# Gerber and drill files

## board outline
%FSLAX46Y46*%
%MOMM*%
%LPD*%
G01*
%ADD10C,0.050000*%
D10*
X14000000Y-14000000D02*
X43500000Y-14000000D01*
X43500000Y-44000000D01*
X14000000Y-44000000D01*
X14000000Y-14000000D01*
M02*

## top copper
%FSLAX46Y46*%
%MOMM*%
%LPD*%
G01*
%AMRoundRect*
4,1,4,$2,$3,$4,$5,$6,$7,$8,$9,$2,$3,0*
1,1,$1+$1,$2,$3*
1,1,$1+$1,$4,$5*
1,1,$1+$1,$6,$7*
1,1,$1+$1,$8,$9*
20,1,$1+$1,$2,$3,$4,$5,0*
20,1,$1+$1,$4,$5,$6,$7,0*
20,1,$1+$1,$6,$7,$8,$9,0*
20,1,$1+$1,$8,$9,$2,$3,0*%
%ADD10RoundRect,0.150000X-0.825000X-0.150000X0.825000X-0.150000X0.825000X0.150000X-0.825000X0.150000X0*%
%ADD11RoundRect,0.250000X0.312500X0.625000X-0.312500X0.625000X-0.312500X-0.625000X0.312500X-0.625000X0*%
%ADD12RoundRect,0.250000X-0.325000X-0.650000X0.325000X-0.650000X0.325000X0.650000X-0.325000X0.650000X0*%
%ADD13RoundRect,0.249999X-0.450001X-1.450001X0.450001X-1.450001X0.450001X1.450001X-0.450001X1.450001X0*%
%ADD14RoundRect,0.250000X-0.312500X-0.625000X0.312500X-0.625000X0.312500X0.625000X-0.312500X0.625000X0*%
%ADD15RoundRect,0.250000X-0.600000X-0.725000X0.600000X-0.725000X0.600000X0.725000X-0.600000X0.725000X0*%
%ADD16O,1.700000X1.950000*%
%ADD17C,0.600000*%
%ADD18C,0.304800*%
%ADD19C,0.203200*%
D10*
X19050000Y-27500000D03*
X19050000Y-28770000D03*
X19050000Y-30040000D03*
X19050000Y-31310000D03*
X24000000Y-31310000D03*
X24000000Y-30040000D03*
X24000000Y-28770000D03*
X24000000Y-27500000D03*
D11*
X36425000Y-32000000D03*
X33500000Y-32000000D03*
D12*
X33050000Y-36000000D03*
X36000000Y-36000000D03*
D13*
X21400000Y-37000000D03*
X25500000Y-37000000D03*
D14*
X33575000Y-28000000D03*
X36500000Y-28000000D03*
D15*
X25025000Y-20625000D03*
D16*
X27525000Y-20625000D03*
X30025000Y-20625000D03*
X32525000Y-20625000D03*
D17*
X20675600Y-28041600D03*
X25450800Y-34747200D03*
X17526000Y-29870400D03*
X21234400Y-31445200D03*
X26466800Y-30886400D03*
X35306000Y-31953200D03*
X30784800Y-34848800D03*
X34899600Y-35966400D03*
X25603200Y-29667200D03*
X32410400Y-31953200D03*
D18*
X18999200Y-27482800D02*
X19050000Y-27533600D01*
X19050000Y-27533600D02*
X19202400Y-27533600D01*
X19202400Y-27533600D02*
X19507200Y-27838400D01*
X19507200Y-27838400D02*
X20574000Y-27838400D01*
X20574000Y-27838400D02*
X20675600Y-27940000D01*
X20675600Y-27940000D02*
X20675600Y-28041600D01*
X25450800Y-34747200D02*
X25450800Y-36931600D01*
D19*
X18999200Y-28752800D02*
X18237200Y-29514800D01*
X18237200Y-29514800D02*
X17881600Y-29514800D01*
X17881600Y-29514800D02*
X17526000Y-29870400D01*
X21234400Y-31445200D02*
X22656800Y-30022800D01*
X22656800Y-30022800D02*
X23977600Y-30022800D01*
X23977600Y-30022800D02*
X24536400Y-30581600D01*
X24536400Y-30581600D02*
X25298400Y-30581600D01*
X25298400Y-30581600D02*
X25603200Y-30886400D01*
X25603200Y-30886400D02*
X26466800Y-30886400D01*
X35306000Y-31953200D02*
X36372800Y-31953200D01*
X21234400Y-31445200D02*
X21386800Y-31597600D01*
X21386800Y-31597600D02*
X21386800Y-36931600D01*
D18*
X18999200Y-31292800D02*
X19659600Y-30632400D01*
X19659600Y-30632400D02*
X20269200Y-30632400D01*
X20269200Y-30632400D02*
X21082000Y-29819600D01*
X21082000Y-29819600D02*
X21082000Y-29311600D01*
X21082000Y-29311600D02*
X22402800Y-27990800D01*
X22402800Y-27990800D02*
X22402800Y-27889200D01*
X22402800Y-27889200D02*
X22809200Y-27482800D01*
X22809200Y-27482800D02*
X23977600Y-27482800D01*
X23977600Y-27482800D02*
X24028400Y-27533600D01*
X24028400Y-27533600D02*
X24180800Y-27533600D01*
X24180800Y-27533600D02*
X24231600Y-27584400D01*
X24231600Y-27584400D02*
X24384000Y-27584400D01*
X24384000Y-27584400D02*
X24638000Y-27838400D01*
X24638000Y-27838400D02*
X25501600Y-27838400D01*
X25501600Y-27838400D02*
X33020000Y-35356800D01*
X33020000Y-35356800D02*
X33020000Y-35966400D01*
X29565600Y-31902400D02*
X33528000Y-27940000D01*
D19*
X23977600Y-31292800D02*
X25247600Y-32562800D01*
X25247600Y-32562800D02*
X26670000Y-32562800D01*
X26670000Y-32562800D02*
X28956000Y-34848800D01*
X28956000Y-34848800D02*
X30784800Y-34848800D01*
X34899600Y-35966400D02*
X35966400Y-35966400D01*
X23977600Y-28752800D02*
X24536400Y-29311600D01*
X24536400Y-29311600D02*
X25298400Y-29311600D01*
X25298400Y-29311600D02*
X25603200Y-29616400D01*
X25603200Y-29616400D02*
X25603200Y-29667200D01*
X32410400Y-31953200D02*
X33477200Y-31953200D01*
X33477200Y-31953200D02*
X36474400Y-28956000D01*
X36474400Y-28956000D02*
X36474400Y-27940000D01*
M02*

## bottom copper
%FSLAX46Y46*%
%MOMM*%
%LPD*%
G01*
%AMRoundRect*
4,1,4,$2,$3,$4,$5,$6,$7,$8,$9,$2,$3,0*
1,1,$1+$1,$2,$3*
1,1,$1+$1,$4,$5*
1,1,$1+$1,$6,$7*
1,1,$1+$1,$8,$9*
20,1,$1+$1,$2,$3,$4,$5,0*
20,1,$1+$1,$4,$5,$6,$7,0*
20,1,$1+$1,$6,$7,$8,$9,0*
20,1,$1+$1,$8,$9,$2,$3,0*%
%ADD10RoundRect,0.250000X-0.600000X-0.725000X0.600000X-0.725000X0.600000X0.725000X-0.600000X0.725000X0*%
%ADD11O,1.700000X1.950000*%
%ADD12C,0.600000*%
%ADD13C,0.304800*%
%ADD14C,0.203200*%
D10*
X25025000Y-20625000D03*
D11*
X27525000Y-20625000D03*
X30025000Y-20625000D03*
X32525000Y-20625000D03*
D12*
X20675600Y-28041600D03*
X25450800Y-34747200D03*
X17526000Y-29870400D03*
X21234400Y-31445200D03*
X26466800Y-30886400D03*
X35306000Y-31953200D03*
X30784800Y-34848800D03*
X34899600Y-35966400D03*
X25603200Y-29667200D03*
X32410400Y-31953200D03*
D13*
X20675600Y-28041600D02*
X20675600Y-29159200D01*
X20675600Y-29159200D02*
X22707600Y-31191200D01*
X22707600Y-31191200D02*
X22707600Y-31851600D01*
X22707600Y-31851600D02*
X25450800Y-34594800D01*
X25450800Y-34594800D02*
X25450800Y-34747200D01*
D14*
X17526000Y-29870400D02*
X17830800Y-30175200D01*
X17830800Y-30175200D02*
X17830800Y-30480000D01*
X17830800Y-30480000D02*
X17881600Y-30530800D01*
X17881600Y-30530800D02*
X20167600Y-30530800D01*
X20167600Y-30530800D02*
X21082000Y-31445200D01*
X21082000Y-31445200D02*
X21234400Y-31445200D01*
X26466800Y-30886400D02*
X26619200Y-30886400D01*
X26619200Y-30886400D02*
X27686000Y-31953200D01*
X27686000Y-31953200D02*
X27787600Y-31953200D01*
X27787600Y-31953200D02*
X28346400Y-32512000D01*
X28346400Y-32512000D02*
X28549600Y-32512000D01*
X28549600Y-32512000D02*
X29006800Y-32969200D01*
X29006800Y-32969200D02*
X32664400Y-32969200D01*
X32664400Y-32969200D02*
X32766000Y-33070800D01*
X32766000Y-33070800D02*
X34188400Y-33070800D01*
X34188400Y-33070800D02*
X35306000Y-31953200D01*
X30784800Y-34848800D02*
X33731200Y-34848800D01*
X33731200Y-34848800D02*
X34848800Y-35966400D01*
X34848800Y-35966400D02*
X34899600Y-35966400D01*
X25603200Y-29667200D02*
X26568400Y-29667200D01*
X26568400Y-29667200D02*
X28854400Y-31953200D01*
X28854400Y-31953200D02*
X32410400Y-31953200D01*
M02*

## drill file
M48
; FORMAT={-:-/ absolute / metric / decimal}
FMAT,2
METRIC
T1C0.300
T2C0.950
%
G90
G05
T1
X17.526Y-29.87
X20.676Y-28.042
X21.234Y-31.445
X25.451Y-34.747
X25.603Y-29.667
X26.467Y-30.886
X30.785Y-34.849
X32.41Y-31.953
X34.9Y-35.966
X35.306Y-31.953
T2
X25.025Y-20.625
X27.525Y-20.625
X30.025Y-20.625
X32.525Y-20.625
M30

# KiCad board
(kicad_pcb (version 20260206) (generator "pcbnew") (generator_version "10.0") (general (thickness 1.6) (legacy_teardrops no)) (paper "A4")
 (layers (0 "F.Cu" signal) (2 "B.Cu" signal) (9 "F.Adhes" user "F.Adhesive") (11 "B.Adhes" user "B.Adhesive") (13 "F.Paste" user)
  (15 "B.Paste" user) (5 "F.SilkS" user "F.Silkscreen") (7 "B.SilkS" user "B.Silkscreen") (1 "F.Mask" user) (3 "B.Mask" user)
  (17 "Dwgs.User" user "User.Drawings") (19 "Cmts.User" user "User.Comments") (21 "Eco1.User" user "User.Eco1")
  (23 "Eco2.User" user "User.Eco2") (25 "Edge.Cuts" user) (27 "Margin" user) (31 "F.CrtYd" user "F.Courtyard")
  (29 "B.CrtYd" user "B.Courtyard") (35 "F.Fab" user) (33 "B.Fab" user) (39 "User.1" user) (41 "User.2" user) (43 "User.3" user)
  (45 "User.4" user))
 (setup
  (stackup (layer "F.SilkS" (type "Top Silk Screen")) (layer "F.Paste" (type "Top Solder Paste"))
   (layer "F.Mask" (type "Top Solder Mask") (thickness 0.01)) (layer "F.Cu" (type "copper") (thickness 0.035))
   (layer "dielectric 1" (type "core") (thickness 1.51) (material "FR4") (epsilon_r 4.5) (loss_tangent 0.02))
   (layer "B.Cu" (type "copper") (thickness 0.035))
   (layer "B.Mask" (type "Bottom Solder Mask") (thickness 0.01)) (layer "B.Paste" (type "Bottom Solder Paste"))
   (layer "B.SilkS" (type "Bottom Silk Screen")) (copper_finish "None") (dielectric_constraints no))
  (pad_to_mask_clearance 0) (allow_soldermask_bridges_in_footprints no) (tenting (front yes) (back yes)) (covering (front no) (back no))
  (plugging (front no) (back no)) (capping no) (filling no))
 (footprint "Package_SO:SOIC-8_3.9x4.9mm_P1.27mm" (layer "F.Cu") (at 21.525 29.405)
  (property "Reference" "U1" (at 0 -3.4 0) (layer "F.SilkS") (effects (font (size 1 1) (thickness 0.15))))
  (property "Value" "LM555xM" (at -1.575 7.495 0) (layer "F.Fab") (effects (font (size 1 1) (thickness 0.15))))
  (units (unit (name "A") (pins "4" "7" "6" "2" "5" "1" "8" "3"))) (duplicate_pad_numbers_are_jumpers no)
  (pad "1" smd roundrect (at -2.475 -1.905) (size 1.95 0.6) (layers "F.Cu" "F.Mask" "F.Paste") (roundrect_rratio 0.25) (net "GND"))
  (pad "2" smd roundrect (at -2.475 -0.635) (size 1.95 0.6) (layers "F.Cu" "F.Mask" "F.Paste") (roundrect_rratio 0.25)
   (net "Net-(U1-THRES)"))
  (pad "3" smd roundrect (at -2.475 0.635) (size 1.95 0.6) (layers "F.Cu" "F.Mask" "F.Paste") (roundrect_rratio 0.25) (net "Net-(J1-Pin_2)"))
  (pad "4" smd roundrect (at -2.475 1.905) (size 1.95 0.6) (layers "F.Cu" "F.Mask" "F.Paste") (roundrect_rratio 0.25) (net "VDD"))
  (pad "5" smd roundrect (at 2.475 1.905) (size 1.95 0.6) (layers "F.Cu" "F.Mask" "F.Paste") (roundrect_rratio 0.25) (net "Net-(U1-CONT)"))
  (pad "6" smd roundrect (at 2.475 0.635) (size 1.95 0.6) (layers "F.Cu" "F.Mask" "F.Paste") (roundrect_rratio 0.25) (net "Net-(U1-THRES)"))
  (pad "7" smd roundrect (at 2.475 -0.635) (size 1.95 0.6) (layers "F.Cu" "F.Mask" "F.Paste") (roundrect_rratio 0.25) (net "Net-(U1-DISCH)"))
  (pad "8" smd roundrect (at 2.475 -1.905) (size 1.95 0.6) (layers "F.Cu" "F.Mask" "F.Paste") (roundrect_rratio 0.25) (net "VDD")))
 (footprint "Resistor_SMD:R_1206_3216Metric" (layer "F.Cu") (at 34.9625 32 180)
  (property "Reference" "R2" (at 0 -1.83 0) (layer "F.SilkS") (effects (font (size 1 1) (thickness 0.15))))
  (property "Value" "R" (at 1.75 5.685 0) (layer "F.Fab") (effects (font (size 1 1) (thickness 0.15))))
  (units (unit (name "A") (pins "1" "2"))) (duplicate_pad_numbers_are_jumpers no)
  (pad "1" smd roundrect (at -1.4625 0 180) (size 1.125 1.75) (layers "F.Cu" "F.Mask" "F.Paste") (roundrect_rratio 0.222222)
   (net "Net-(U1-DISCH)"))
  (pad "2" smd roundrect (at 1.4625 0 180) (size 1.125 1.75) (layers "F.Cu" "F.Mask" "F.Paste") (roundrect_rratio 0.222222)
   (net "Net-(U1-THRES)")))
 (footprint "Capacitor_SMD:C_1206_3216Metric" (layer "F.Cu") (at 34.525 36)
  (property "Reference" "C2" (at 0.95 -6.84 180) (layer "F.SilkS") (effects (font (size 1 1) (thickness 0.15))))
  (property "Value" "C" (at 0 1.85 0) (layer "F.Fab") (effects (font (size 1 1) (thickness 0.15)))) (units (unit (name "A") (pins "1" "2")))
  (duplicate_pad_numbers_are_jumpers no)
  (pad "1" smd roundrect (at -1.475 0) (size 1.15 1.8) (layers "F.Cu" "F.Mask" "F.Paste") (roundrect_rratio 0.217391) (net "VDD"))
  (pad "2" smd roundrect (at 1.475 0) (size 1.15 1.8) (layers "F.Cu" "F.Mask" "F.Paste") (roundrect_rratio 0.217391) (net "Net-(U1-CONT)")))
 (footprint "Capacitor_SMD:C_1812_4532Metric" (layer "F.Cu") (at 23.45 37)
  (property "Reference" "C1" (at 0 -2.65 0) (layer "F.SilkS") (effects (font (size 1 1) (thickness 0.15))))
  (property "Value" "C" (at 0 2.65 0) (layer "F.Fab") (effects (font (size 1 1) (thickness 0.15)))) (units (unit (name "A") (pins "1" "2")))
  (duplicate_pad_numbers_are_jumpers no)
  (pad "1" smd roundrect (at -2.05 0) (size 1.4 3.4) (layers "F.Cu" "F.Mask" "F.Paste") (roundrect_rratio 0.178571) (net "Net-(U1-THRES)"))
  (pad "2" smd roundrect (at 2.05 0) (size 1.4 3.4) (layers "F.Cu" "F.Mask" "F.Paste") (roundrect_rratio 0.178571) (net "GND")))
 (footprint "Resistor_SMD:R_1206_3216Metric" (layer "F.Cu") (at 35.0375 28)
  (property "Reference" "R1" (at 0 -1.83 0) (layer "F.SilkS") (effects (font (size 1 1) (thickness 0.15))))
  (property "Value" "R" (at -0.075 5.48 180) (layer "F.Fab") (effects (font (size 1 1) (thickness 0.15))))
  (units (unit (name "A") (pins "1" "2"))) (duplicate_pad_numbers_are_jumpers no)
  (pad "1" smd roundrect (at -1.4625 0) (size 1.125 1.75) (layers "F.Cu" "F.Mask" "F.Paste") (roundrect_rratio 0.222222) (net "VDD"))
  (pad "2" smd roundrect (at 1.4625 0) (size 1.125 1.75) (layers "F.Cu" "F.Mask" "F.Paste") (roundrect_rratio 0.222222)
   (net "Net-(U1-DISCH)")))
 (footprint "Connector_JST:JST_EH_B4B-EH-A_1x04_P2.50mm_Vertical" (layer "F.Cu") (at 25.025 20.625)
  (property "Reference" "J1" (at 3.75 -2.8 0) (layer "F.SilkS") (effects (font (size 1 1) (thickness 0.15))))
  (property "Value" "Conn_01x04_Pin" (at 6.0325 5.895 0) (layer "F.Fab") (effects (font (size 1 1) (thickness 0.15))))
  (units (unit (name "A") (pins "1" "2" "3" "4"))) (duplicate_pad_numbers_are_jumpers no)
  (pad "1" thru_hole roundrect (at 0 0) (size 1.7 1.95) (drill 0.95) (layers "*.Cu" "*.Mask") (remove_unused_layers no)
   (roundrect_rratio 0.147059) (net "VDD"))
  (pad "2" thru_hole oval (at 2.5 0) (size 1.7 1.95) (drill 0.95) (layers "*.Cu" "*.Mask") (remove_unused_layers no) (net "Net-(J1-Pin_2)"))
  (pad "3" thru_hole oval (at 5 0) (size 1.7 1.95) (drill 0.95) (layers "*.Cu" "*.Mask") (remove_unused_layers no)
   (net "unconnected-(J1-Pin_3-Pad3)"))
  (pad "4" thru_hole oval (at 7.5 0) (size 1.7 1.95) (drill 0.95) (layers "*.Cu" "*.Mask") (remove_unused_layers no) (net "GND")))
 (gr_rect (start 14 14) (end 43.5 44) (stroke (width 0.05) (type default)) (fill no) (layer "Edge.Cuts"))
 (segment (start 18.9992 27.4828) (end 19.05 27.5336) (width 0.3048) (layer "F.Cu") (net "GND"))
 (segment (start 19.05 27.5336) (end 19.2024 27.5336) (width 0.3048) (layer "F.Cu") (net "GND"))
 (segment (start 19.2024 27.5336) (end 19.5072 27.8384) (width 0.3048) (layer "F.Cu") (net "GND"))
 (segment (start 19.5072 27.8384) (end 20.574 27.8384) (width 0.3048) (layer "F.Cu") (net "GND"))
 (segment (start 20.574 27.8384) (end 20.6756 27.94) (width 0.3048) (layer "F.Cu") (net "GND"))
 (segment (start 20.6756 27.94) (end 20.6756 28.0416) (width 0.3048) (layer "F.Cu") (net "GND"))
 (segment (start 25.4508 34.7472) (end 25.4508 36.9316) (width 0.3048) (layer "F.Cu") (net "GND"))
 (segment (start 20.6756 28.0416) (end 20.6756 29.1592) (width 0.3048) (layer "B.Cu") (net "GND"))
 (segment (start 20.6756 29.1592) (end 22.7076 31.1912) (width 0.3048) (layer "B.Cu") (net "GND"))
 (segment (start 22.7076 31.1912) (end 22.7076 31.8516) (width 0.3048) (layer "B.Cu") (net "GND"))
 (segment (start 22.7076 31.8516) (end 25.4508 34.5948) (width 0.3048) (layer "B.Cu") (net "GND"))
 (segment (start 25.4508 34.5948) (end 25.4508 34.7472) (width 0.3048) (layer "B.Cu") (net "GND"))
 (via (at 20.6756 28.0416) (size 0.6) (drill 0.3) (layers "F.Cu" "B.Cu") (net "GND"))
 (via (at 25.4508 34.7472) (size 0.6) (drill 0.3) (layers "F.Cu" "B.Cu") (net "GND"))
 (segment (start 18.9992 28.7528) (end 18.2372 29.5148) (width 0.2032) (layer "F.Cu") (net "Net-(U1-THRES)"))
 (segment (start 18.2372 29.5148) (end 17.8816 29.5148) (width 0.2032) (layer "F.Cu") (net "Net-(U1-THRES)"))
 (segment (start 17.8816 29.5148) (end 17.526 29.8704) (width 0.2032) (layer "F.Cu") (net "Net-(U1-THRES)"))
 (segment (start 21.2344 31.4452) (end 22.6568 30.0228) (width 0.2032) (layer "F.Cu") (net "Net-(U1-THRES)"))
 (segment (start 22.6568 30.0228) (end 23.9776 30.0228) (width 0.2032) (layer "F.Cu") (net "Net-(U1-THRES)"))
 (segment (start 17.526 29.8704) (end 17.8308 30.1752) (width 0.2032) (layer "B.Cu") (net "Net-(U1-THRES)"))
 (segment (start 17.8308 30.1752) (end 17.8308 30.48) (width 0.2032) (layer "B.Cu") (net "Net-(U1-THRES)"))
 (segment (start 17.8308 30.48) (end 17.8816 30.5308) (width 0.2032) (layer "B.Cu") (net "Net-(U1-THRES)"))
 (segment (start 17.8816 30.5308) (end 20.1676 30.5308) (width 0.2032) (layer "B.Cu") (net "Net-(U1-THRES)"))
 (segment (start 20.1676 30.5308) (end 21.082 31.4452) (width 0.2032) (layer "B.Cu") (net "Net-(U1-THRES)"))
 (segment (start 21.082 31.4452) (end 21.2344 31.4452) (width 0.2032) (layer "B.Cu") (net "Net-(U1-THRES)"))
 (via (at 17.526 29.8704) (size 0.6) (drill 0.3) (layers "F.Cu" "B.Cu") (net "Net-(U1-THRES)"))
 (via (at 21.2344 31.4452) (size 0.6) (drill 0.3) (layers "F.Cu" "B.Cu") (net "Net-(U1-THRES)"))
 (segment (start 23.9776 30.0228) (end 24.5364 30.5816) (width 0.2032) (layer "F.Cu") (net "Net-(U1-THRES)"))
 (segment (start 24.5364 30.5816) (end 25.2984 30.5816) (width 0.2032) (layer "F.Cu") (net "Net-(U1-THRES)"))
 (segment (start 25.2984 30.5816) (end 25.6032 30.8864) (width 0.2032) (layer "F.Cu") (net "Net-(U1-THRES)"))
 (segment (start 25.6032 30.8864) (end 26.4668 30.8864) (width 0.2032) (layer "F.Cu") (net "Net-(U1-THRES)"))
 (segment (start 35.306 31.9532) (end 36.3728 31.9532) (width 0.2032) (layer "F.Cu") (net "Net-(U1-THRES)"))
 (segment (start 26.4668 30.8864) (end 26.6192 30.8864) (width 0.2032) (layer "B.Cu") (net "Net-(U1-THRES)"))
 (segment (start 26.6192 30.8864) (end 27.686 31.9532) (width 0.2032) (layer "B.Cu") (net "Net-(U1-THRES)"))
 (segment (start 27.686 31.9532) (end 27.7876 31.9532) (width 0.2032) (layer "B.Cu") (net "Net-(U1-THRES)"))
 (segment (start 27.7876 31.9532) (end 28.3464 32.512) (width 0.2032) (layer "B.Cu") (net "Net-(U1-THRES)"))
 (segment (start 28.3464 32.512) (end 28.5496 32.512) (width 0.2032) (layer "B.Cu") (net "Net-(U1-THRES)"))
 (segment (start 28.5496 32.512) (end 29.0068 32.9692) (width 0.2032) (layer "B.Cu") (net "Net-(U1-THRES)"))
 (segment (start 29.0068 32.9692) (end 32.6644 32.9692) (width 0.2032) (layer "B.Cu") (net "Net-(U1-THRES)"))
 (segment (start 32.6644 32.9692) (end 32.766 33.0708) (width 0.2032) (layer "B.Cu") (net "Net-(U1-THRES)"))
 (segment (start 32.766 33.0708) (end 34.1884 33.0708) (width 0.2032) (layer "B.Cu") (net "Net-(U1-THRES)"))
 (segment (start 34.1884 33.0708) (end 35.306 31.9532) (width 0.2032) (layer "B.Cu") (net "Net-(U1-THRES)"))
 (via (at 26.4668 30.8864) (size 0.6) (drill 0.3) (layers "F.Cu" "B.Cu") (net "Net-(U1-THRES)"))
 (via (at 35.306 31.9532) (size 0.6) (drill 0.3) (layers "F.Cu" "B.Cu") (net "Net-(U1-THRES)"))
 (segment (start 21.2344 31.4452) (end 21.3868 31.5976) (width 0.2032) (layer "F.Cu") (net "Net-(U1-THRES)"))
 (segment (start 21.3868 31.5976) (end 21.3868 36.9316) (width 0.2032) (layer "F.Cu") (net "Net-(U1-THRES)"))
 (segment (start 18.9992 31.2928) (end 19.6596 30.6324) (width 0.3048) (layer "F.Cu") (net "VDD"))
 (segment (start 19.6596 30.6324) (end 20.2692 30.6324) (width 0.3048) (layer "F.Cu") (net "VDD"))
 (segment (start 20.2692 30.6324) (end 21.082 29.8196) (width 0.3048) (layer "F.Cu") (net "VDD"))
 (segment (start 21.082 29.8196) (end 21.082 29.3116) (width 0.3048) (layer "F.Cu") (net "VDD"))
 (segment (start 21.082 29.3116) (end 22.4028 27.9908) (width 0.3048) (layer "F.Cu") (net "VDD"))
 (segment (start 22.4028 27.9908) (end 22.4028 27.8892) (width 0.3048) (layer "F.Cu") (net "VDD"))
 (segment (start 22.4028 27.8892) (end 22.8092 27.4828) (width 0.3048) (layer "F.Cu") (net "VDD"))
 (segment (start 22.8092 27.4828) (end 23.9776 27.4828) (width 0.3048) (layer "F.Cu") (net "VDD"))
 (segment (start 23.9776 27.4828) (end 24.0284 27.5336) (width 0.3048) (layer "F.Cu") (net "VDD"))
 (segment (start 24.0284 27.5336) (end 24.1808 27.5336) (width 0.3048) (layer "F.Cu") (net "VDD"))
 (segment (start 24.1808 27.5336) (end 24.2316 27.5844) (width 0.3048) (layer "F.Cu") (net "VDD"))
 (segment (start 24.2316 27.5844) (end 24.384 27.5844) (width 0.3048) (layer "F.Cu") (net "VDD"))
 (segment (start 24.384 27.5844) (end 24.638 27.8384) (width 0.3048) (layer "F.Cu") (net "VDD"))
 (segment (start 24.638 27.8384) (end 25.5016 27.8384) (width 0.3048) (layer "F.Cu") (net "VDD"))
 (segment (start 25.5016 27.8384) (end 33.02 35.3568) (width 0.3048) (layer "F.Cu") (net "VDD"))
 (segment (start 33.02 35.3568) (end 33.02 35.9664) (width 0.3048) (layer "F.Cu") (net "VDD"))
 (segment (start 29.5656 31.9024) (end 33.528 27.94) (width 0.3048) (layer "F.Cu") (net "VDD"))
 (segment (start 23.9776 31.2928) (end 25.2476 32.5628) (width 0.2032) (layer "F.Cu") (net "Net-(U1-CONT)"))
 (segment (start 25.2476 32.5628) (end 26.67 32.5628) (width 0.2032) (layer "F.Cu") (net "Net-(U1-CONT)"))
 (segment (start 26.67 32.5628) (end 28.956 34.8488) (width 0.2032) (layer "F.Cu") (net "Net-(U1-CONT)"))
 (segment (start 28.956 34.8488) (end 30.7848 34.8488) (width 0.2032) (layer "F.Cu") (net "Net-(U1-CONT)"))
 (segment (start 34.8996 35.9664) (end 35.9664 35.9664) (width 0.2032) (layer "F.Cu") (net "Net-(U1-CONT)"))
 (segment (start 30.7848 34.8488) (end 33.7312 34.8488) (width 0.2032) (layer "B.Cu") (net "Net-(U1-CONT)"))
 (segment (start 33.7312 34.8488) (end 34.8488 35.9664) (width 0.2032) (layer "B.Cu") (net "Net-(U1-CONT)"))
 (segment (start 34.8488 35.9664) (end 34.8996 35.9664) (width 0.2032) (layer "B.Cu") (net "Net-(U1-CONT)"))
 (via (at 30.7848 34.8488) (size 0.6) (drill 0.3) (layers "F.Cu" "B.Cu") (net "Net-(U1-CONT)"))
 (via (at 34.8996 35.9664) (size 0.6) (drill 0.3) (layers "F.Cu" "B.Cu") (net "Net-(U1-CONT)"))
 (segment (start 23.9776 28.7528) (end 24.5364 29.3116) (width 0.2032) (layer "F.Cu") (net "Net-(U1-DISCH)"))
 (segment (start 24.5364 29.3116) (end 25.2984 29.3116) (width 0.2032) (layer "F.Cu") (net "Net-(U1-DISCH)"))
 (segment (start 25.2984 29.3116) (end 25.6032 29.6164) (width 0.2032) (layer "F.Cu") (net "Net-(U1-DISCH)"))
 (segment (start 25.6032 29.6164) (end 25.6032 29.6672) (width 0.2032) (layer "F.Cu") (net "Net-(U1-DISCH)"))
 (segment (start 32.4104 31.9532) (end 33.4772 31.9532) (width 0.2032) (layer "F.Cu") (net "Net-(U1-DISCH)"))
 (segment (start 25.6032 29.6672) (end 26.5684 29.6672) (width 0.2032) (layer "B.Cu") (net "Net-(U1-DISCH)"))
 (segment (start 26.5684 29.6672) (end 28.8544 31.9532) (width 0.2032) (layer "B.Cu") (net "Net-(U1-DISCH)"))
 (segment (start 28.8544 31.9532) (end 32.4104 31.9532) (width 0.2032) (layer "B.Cu") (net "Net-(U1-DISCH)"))
 (via (at 25.6032 29.6672) (size 0.6) (drill 0.3) (layers "F.Cu" "B.Cu") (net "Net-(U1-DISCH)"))
 (via (at 32.4104 31.9532) (size 0.6) (drill 0.3) (layers "F.Cu" "B.Cu") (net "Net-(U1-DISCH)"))
 (segment (start 33.4772 31.9532) (end 36.4744 28.956) (width 0.2032) (layer "F.Cu") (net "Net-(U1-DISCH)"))
 (segment (start 36.4744 28.956) (end 36.4744 27.94) (width 0.2032) (layer "F.Cu") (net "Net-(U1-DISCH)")))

